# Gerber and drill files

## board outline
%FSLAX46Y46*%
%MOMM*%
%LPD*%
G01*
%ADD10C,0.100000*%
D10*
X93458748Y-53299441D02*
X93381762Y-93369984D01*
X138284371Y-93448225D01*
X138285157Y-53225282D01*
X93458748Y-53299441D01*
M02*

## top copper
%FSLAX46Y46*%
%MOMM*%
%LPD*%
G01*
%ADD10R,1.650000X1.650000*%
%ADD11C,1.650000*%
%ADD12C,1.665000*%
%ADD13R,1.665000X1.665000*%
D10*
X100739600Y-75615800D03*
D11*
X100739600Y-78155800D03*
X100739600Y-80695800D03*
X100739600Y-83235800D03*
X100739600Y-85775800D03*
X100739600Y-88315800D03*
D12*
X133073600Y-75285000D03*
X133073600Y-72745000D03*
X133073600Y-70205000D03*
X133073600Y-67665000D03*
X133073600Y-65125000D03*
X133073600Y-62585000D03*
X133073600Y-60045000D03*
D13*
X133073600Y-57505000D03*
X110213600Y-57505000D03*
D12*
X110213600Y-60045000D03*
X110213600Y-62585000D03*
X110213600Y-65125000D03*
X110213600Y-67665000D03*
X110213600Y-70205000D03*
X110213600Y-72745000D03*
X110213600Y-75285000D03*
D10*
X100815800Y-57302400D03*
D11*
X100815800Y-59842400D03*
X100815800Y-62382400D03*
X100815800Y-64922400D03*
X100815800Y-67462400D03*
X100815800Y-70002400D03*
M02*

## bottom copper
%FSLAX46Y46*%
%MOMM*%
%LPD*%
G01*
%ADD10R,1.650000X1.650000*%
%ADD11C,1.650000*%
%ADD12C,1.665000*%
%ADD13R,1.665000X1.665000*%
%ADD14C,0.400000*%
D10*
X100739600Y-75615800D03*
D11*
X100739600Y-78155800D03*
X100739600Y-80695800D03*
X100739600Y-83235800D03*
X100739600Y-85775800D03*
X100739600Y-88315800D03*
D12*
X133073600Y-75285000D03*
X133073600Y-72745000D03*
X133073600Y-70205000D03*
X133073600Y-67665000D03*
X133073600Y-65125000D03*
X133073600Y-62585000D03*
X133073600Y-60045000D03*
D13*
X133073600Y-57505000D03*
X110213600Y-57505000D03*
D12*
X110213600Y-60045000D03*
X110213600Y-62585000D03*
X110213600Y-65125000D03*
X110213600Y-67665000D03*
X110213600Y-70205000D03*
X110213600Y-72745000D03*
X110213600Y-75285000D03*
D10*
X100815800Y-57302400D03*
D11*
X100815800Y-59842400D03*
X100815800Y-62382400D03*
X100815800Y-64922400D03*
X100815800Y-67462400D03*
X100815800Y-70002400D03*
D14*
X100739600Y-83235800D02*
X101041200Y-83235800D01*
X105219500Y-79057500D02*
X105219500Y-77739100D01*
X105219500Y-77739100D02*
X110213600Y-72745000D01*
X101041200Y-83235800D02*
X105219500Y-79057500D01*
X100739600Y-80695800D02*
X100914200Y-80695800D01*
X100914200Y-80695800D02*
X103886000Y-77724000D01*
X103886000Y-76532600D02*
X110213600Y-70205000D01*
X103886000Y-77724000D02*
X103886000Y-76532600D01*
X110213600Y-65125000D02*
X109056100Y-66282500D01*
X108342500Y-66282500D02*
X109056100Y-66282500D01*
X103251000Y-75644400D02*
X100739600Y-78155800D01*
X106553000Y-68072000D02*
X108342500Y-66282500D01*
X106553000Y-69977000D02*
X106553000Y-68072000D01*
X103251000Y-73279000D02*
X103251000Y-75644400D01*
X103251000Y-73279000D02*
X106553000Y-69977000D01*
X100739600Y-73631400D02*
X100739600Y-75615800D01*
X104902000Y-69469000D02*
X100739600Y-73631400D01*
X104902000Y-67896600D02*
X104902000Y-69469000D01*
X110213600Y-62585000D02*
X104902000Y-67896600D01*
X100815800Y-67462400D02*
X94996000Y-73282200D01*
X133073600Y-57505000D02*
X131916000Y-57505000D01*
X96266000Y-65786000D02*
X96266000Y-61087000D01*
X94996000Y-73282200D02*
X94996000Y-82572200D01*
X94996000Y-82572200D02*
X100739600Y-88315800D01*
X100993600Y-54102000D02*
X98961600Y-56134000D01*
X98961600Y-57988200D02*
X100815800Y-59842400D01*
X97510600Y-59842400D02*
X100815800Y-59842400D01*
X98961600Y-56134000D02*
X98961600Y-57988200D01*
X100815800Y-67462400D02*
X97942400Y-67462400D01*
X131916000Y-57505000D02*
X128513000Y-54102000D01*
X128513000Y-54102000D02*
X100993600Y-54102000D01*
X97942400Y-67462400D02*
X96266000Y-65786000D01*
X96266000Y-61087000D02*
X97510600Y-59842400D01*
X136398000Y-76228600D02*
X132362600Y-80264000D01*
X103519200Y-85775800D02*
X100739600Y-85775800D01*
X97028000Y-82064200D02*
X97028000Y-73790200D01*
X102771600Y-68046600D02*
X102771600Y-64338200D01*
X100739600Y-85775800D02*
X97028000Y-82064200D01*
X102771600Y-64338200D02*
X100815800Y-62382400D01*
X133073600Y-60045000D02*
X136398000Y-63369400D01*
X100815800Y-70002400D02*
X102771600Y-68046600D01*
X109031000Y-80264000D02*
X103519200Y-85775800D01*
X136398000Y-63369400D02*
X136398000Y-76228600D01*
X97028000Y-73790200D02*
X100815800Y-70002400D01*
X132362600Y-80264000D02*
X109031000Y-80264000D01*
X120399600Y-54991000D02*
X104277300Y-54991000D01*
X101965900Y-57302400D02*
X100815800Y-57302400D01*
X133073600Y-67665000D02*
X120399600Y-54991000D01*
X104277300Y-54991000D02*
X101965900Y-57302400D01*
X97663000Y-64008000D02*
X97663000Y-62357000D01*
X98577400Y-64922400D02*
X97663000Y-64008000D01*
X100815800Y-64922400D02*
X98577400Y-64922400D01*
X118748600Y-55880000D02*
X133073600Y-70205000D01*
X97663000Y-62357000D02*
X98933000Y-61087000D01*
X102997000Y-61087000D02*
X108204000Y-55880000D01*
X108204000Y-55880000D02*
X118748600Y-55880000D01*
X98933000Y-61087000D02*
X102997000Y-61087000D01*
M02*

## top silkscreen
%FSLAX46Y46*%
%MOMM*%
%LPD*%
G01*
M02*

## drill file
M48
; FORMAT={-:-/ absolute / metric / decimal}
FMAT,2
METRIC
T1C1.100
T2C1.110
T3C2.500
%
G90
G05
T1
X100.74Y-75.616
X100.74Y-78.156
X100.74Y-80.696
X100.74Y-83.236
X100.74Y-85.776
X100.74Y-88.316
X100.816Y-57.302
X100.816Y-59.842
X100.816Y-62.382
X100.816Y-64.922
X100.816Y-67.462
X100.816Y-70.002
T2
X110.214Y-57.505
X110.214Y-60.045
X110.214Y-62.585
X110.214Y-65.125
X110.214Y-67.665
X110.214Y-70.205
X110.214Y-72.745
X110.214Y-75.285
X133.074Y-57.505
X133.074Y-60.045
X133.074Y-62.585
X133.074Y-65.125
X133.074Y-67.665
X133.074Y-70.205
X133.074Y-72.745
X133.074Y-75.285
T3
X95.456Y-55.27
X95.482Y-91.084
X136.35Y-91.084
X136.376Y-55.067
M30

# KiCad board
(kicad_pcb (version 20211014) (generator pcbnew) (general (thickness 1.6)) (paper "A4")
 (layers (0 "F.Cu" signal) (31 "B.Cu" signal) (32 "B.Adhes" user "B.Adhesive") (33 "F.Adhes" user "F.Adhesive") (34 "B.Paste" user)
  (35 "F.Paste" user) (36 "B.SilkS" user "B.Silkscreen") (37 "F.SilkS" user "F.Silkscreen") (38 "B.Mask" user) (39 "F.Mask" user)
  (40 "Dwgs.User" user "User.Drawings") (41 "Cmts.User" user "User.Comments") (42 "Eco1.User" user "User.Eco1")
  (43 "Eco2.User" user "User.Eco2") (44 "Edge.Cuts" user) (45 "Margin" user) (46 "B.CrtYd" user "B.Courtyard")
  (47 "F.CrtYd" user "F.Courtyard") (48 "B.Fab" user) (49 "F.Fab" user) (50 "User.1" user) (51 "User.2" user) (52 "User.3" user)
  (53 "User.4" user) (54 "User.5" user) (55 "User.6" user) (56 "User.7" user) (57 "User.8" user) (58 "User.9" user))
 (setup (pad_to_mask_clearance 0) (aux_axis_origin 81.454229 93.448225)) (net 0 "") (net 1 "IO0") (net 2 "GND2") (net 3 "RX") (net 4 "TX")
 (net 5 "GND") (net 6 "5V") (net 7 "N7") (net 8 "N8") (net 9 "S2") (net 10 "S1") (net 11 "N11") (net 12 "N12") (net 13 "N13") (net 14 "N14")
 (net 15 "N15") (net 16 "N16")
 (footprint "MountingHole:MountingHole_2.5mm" (layer "B.Cu") (at 95.4564 55.2704 180)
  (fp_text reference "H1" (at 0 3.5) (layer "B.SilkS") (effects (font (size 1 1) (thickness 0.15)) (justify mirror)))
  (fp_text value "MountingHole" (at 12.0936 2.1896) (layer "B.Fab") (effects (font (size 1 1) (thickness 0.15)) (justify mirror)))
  (pad "" np_thru_hole circle (at 0 0 180) (size 2.5 2.5) (drill 2.5) (layers *.Cu *.Mask)))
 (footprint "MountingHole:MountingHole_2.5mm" (layer "B.Cu") (at 136.3758 55.0672 180)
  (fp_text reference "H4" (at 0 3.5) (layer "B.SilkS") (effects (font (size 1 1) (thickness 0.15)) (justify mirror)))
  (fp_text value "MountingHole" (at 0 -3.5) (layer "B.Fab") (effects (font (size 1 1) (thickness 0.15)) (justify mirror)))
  (pad "" np_thru_hole circle (at 0 0 180) (size 2.5 2.5) (drill 2.5) (layers *.Cu *.Mask)))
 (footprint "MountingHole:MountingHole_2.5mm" (layer "B.Cu") (at 136.3504 91.0844 180)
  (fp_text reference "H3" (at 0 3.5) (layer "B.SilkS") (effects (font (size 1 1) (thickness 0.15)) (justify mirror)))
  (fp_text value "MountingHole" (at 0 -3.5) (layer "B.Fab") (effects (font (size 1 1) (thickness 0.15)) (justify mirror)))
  (pad "" np_thru_hole circle (at 0 0 180) (size 2.5 2.5) (drill 2.5) (layers *.Cu *.Mask)))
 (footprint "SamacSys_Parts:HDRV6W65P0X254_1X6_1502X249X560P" (layer "B.Cu") (at 100.7396 75.6158 -90)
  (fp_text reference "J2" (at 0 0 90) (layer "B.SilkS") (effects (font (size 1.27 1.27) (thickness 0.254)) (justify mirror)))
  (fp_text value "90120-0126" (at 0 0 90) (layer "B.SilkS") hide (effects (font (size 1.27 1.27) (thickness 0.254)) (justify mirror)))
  (pad "1" thru_hole rect (at 0 0 180) (size 1.65 1.65) (drill 1.1) (layers *.Cu *.Mask "B.SilkS") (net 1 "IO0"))
  (pad "2" thru_hole circle (at 2.54 0 180) (size 1.65 1.65) (drill 1.1) (layers *.Cu *.Mask "B.SilkS") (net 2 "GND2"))
  (pad "3" thru_hole circle (at 5.08 0 180) (size 1.65 1.65) (drill 1.1) (layers *.Cu *.Mask "B.SilkS") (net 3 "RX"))
  (pad "4" thru_hole circle (at 7.62 0 180) (size 1.65 1.65) (drill 1.1) (layers *.Cu *.Mask "B.SilkS") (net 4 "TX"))
  (pad "5" thru_hole circle (at 10.16 0 180) (size 1.65 1.65) (drill 1.1) (layers *.Cu *.Mask "B.SilkS") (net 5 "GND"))
  (pad "6" thru_hole circle (at 12.7 0 180) (size 1.65 1.65) (drill 1.1) (layers *.Cu *.Mask "B.SilkS") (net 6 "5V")))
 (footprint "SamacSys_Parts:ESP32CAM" (layer "B.Cu") (at 133.0736 75.285 180)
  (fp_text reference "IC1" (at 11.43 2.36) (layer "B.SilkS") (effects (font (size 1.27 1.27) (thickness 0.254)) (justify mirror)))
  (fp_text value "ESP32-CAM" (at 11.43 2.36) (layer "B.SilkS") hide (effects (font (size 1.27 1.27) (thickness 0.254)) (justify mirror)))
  (pad "1" thru_hole circle (at 0 0 90) (size 1.665 1.665) (drill 1.11) (layers *.Cu *.Mask "B.SilkS") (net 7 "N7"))
  (pad "2" thru_hole circle (at 0 2.54 90) (size 1.665 1.665) (drill 1.11) (layers *.Cu *.Mask "B.SilkS") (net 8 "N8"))
  (pad "3" thru_hole circle (at 0 5.08 90) (size 1.665 1.665) (drill 1.11) (layers *.Cu *.Mask "B.SilkS") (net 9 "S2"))
  (pad "4" thru_hole circle (at 0 7.62 90) (size 1.665 1.665) (drill 1.11) (layers *.Cu *.Mask "B.SilkS") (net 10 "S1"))
  (pad "5" thru_hole circle (at 0 10.16 90) (size 1.665 1.665) (drill 1.11) (layers *.Cu *.Mask "B.SilkS") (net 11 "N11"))
  (pad "6" thru_hole circle (at 0 12.7 90) (size 1.665 1.665) (drill 1.11) (layers *.Cu *.Mask "B.SilkS") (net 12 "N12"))
  (pad "7" thru_hole circle (at 0 15.24 90) (size 1.665 1.665) (drill 1.11) (layers *.Cu *.Mask "B.SilkS") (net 5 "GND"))
  (pad "8" thru_hole rect (at 0 17.78 90) (size 1.665 1.665) (drill 1.11) (layers *.Cu *.Mask "B.SilkS") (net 6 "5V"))
  (pad "9" thru_hole rect (at 22.86 17.78 90) (size 1.665 1.665) (drill 1.11) (layers *.Cu *.Mask "B.SilkS") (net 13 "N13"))
  (pad "10" thru_hole circle (at 22.86 15.24 90) (size 1.665 1.665) (drill 1.11) (layers *.Cu *.Mask "B.SilkS") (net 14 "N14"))
  (pad "11" thru_hole circle (at 22.86 12.7 90) (size 1.665 1.665) (drill 1.11) (layers *.Cu *.Mask "B.SilkS") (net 1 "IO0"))
  (pad "12" thru_hole circle (at 22.86 10.16 90) (size 1.665 1.665) (drill 1.11) (layers *.Cu *.Mask "B.SilkS") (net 2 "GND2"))
  (pad "13" thru_hole circle (at 22.86 7.62 90) (size 1.665 1.665) (drill 1.11) (layers *.Cu *.Mask "B.SilkS") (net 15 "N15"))
  (pad "14" thru_hole circle (at 22.86 5.08 90) (size 1.665 1.665) (drill 1.11) (layers *.Cu *.Mask "B.SilkS") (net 3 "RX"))
  (pad "15" thru_hole circle (at 22.86 2.54 90) (size 1.665 1.665) (drill 1.11) (layers *.Cu *.Mask "B.SilkS") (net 4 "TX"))
  (pad "16" thru_hole circle (at 22.86 0 90) (size 1.665 1.665) (drill 1.11) (layers *.Cu *.Mask "B.SilkS") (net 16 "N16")))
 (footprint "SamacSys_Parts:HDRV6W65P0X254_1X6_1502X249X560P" (layer "B.Cu") (at 100.8158 57.3024 -90)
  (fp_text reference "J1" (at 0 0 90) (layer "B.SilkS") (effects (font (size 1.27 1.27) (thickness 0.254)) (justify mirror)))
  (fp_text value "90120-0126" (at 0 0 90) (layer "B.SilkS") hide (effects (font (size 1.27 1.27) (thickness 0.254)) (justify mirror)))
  (pad "1" thru_hole rect (at 0 0 180) (size 1.65 1.65) (drill 1.1) (layers *.Cu *.Mask "B.SilkS") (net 10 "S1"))
  (pad "2" thru_hole circle (at 2.54 0 180) (size 1.65 1.65) (drill 1.1) (layers *.Cu *.Mask "B.SilkS") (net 6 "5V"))
  (pad "3" thru_hole circle (at 5.08 0 180) (size 1.65 1.65) (drill 1.1) (layers *.Cu *.Mask "B.SilkS") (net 5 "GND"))
  (pad "4" thru_hole circle (at 7.62 0 180) (size 1.65 1.65) (drill 1.1) (layers *.Cu *.Mask "B.SilkS") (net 9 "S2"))
  (pad "5" thru_hole circle (at 10.16 0 180) (size 1.65 1.65) (drill 1.1) (layers *.Cu *.Mask "B.SilkS") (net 6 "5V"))
  (pad "6" thru_hole circle (at 12.7 0 180) (size 1.65 1.65) (drill 1.1) (layers *.Cu *.Mask "B.SilkS") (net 5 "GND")))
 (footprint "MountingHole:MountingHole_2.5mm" (layer "B.Cu") (at 95.4818 91.0844 180)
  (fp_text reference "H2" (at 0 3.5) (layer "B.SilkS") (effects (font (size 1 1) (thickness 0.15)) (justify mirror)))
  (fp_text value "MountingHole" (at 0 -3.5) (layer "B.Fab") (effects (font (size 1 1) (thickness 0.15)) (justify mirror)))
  (pad "" np_thru_hole circle (at 0 0 180) (size 2.5 2.5) (drill 2.5) (layers *.Cu *.Mask)))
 (gr_poly
  (pts (xy 93.458748 53.299441) (xy 93.381762 93.369984) (xy 138.284371 93.448225) (xy 138.285157 53.225282)) (layer "Edge.Cuts")
  (width 0.1) (fill none))
 (segment (start 100.7396 83.2358) (end 101.0412 83.2358) (width 0.4) (layer "B.Cu") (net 4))
 (segment (start 105.2195 79.0575) (end 105.2195 77.7391) (width 0.4) (layer "B.Cu") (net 4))
 (segment (start 105.2195 77.7391) (end 110.2136 72.745) (width 0.4) (layer "B.Cu") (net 4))
 (segment (start 101.0412 83.2358) (end 105.2195 79.0575) (width 0.4) (layer "B.Cu") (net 4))
 (segment (start 100.7396 80.6958) (end 100.9142 80.6958) (width 0.4) (layer "B.Cu") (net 3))
 (segment (start 100.9142 80.6958) (end 103.886 77.724) (width 0.4) (layer "B.Cu") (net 3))
 (segment (start 103.886 76.5326) (end 110.2136 70.205) (width 0.4) (layer "B.Cu") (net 3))
 (segment (start 103.886 77.724) (end 103.886 76.5326) (width 0.4) (layer "B.Cu") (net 3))
 (segment (start 110.2136 65.125) (end 109.0561 66.2825) (width 0.4) (layer "B.Cu") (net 2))
 (segment (start 108.3425 66.2825) (end 109.0561 66.2825) (width 0.4) (layer "B.Cu") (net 2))
 (segment (start 103.251 75.6444) (end 100.7396 78.1558) (width 0.4) (layer "B.Cu") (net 2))
 (segment (start 106.553 68.072) (end 108.3425 66.2825) (width 0.4) (layer "B.Cu") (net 2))
 (segment (start 106.553 69.977) (end 106.553 68.072) (width 0.4) (layer "B.Cu") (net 2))
 (segment (start 103.251 73.279) (end 103.251 75.6444) (width 0.4) (layer "B.Cu") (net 2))
 (segment (start 103.251 73.279) (end 106.553 69.977) (width 0.4) (layer "B.Cu") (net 2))
 (segment (start 100.7396 73.6314) (end 100.7396 75.6158) (width 0.4) (layer "B.Cu") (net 1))
 (segment (start 104.902 69.469) (end 100.7396 73.6314) (width 0.4) (layer "B.Cu") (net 1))
 (segment (start 104.902 67.8966) (end 104.902 69.469) (width 0.4) (layer "B.Cu") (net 1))
 (segment (start 110.2136 62.585) (end 104.902 67.8966) (width 0.4) (layer "B.Cu") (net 1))
 (segment (start 100.8158 67.4624) (end 94.996 73.2822) (width 0.4) (layer "B.Cu") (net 6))
 (segment (start 133.0736 57.505) (end 131.916 57.505) (width 0.4) (layer "B.Cu") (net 6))
 (segment (start 96.266 65.786) (end 96.266 61.087) (width 0.4) (layer "B.Cu") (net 6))
 (segment (start 94.996 73.2822) (end 94.996 82.5722) (width 0.4) (layer "B.Cu") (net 6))
 (segment (start 94.996 82.5722) (end 100.7396 88.3158) (width 0.4) (layer "B.Cu") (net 6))
 (segment (start 100.9936 54.102) (end 98.9616 56.134) (width 0.4) (layer "B.Cu") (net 6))
 (segment (start 98.9616 57.9882) (end 100.8158 59.8424) (width 0.4) (layer "B.Cu") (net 6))
 (segment (start 97.5106 59.8424) (end 100.8158 59.8424) (width 0.4) (layer "B.Cu") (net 6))
 (segment (start 98.9616 56.134) (end 98.9616 57.9882) (width 0.4) (layer "B.Cu") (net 6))
 (segment (start 100.8158 67.4624) (end 97.9424 67.4624) (width 0.4) (layer "B.Cu") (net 6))
 (segment (start 131.916 57.505) (end 128.513 54.102) (width 0.4) (layer "B.Cu") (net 6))
 (segment (start 128.513 54.102) (end 100.9936 54.102) (width 0.4) (layer "B.Cu") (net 6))
 (segment (start 97.9424 67.4624) (end 96.266 65.786) (width 0.4) (layer "B.Cu") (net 6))
 (segment (start 96.266 61.087) (end 97.5106 59.8424) (width 0.4) (layer "B.Cu") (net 6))
 (segment (start 136.398 76.2286) (end 132.3626 80.264) (width 0.4) (layer "B.Cu") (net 5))
 (segment (start 103.5192 85.7758) (end 100.7396 85.7758) (width 0.4) (layer "B.Cu") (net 5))
 (segment (start 97.028 82.0642) (end 97.028 73.7902) (width 0.4) (layer "B.Cu") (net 5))
 (segment (start 102.7716 68.0466) (end 102.7716 64.3382) (width 0.4) (layer "B.Cu") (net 5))
 (segment (start 100.7396 85.7758) (end 97.028 82.0642) (width 0.4) (layer "B.Cu") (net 5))
 (segment (start 102.7716 64.3382) (end 100.8158 62.3824) (width 0.4) (layer "B.Cu") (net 5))
 (segment (start 133.0736 60.045) (end 136.398 63.3694) (width 0.4) (layer "B.Cu") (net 5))
 (segment (start 100.8158 70.0024) (end 102.7716 68.0466) (width 0.4) (layer "B.Cu") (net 5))
 (segment (start 109.031 80.264) (end 103.5192 85.7758) (width 0.4) (layer "B.Cu") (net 5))
 (segment (start 136.398 63.3694) (end 136.398 76.2286) (width 0.4) (layer "B.Cu") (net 5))
 (segment (start 97.028 73.7902) (end 100.8158 70.0024) (width 0.4) (layer "B.Cu") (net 5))
 (segment (start 132.3626 80.264) (end 109.031 80.264) (width 0.4) (layer "B.Cu") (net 5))
 (segment (start 120.3996 54.991) (end 104.2773 54.991) (width 0.4) (layer "B.Cu") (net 10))
 (segment (start 101.9659 57.3024) (end 100.8158 57.3024) (width 0.4) (layer "B.Cu") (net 10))
 (segment (start 133.0736 67.665) (end 120.3996 54.991) (width 0.4) (layer "B.Cu") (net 10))
 (segment (start 104.2773 54.991) (end 101.9659 57.3024) (width 0.4) (layer "B.Cu") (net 10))
 (segment (start 97.663 64.008) (end 97.663 62.357) (width 0.4) (layer "B.Cu") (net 9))
 (segment (start 98.5774 64.9224) (end 97.663 64.008) (width 0.4) (layer "B.Cu") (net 9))
 (segment (start 100.8158 64.9224) (end 98.5774 64.9224) (width 0.4) (layer "B.Cu") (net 9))
 (segment (start 118.7486 55.88) (end 133.0736 70.205) (width 0.4) (layer "B.Cu") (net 9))
 (segment (start 97.663 62.357) (end 98.933 61.087) (width 0.4) (layer "B.Cu") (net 9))
 (segment (start 102.997 61.087) (end 108.204 55.88) (width 0.4) (layer "B.Cu") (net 9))
 (segment (start 108.204 55.88) (end 118.7486 55.88) (width 0.4) (layer "B.Cu") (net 9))
 (segment (start 98.933 61.087) (end 102.997 61.087) (width 0.4) (layer "B.Cu") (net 9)))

